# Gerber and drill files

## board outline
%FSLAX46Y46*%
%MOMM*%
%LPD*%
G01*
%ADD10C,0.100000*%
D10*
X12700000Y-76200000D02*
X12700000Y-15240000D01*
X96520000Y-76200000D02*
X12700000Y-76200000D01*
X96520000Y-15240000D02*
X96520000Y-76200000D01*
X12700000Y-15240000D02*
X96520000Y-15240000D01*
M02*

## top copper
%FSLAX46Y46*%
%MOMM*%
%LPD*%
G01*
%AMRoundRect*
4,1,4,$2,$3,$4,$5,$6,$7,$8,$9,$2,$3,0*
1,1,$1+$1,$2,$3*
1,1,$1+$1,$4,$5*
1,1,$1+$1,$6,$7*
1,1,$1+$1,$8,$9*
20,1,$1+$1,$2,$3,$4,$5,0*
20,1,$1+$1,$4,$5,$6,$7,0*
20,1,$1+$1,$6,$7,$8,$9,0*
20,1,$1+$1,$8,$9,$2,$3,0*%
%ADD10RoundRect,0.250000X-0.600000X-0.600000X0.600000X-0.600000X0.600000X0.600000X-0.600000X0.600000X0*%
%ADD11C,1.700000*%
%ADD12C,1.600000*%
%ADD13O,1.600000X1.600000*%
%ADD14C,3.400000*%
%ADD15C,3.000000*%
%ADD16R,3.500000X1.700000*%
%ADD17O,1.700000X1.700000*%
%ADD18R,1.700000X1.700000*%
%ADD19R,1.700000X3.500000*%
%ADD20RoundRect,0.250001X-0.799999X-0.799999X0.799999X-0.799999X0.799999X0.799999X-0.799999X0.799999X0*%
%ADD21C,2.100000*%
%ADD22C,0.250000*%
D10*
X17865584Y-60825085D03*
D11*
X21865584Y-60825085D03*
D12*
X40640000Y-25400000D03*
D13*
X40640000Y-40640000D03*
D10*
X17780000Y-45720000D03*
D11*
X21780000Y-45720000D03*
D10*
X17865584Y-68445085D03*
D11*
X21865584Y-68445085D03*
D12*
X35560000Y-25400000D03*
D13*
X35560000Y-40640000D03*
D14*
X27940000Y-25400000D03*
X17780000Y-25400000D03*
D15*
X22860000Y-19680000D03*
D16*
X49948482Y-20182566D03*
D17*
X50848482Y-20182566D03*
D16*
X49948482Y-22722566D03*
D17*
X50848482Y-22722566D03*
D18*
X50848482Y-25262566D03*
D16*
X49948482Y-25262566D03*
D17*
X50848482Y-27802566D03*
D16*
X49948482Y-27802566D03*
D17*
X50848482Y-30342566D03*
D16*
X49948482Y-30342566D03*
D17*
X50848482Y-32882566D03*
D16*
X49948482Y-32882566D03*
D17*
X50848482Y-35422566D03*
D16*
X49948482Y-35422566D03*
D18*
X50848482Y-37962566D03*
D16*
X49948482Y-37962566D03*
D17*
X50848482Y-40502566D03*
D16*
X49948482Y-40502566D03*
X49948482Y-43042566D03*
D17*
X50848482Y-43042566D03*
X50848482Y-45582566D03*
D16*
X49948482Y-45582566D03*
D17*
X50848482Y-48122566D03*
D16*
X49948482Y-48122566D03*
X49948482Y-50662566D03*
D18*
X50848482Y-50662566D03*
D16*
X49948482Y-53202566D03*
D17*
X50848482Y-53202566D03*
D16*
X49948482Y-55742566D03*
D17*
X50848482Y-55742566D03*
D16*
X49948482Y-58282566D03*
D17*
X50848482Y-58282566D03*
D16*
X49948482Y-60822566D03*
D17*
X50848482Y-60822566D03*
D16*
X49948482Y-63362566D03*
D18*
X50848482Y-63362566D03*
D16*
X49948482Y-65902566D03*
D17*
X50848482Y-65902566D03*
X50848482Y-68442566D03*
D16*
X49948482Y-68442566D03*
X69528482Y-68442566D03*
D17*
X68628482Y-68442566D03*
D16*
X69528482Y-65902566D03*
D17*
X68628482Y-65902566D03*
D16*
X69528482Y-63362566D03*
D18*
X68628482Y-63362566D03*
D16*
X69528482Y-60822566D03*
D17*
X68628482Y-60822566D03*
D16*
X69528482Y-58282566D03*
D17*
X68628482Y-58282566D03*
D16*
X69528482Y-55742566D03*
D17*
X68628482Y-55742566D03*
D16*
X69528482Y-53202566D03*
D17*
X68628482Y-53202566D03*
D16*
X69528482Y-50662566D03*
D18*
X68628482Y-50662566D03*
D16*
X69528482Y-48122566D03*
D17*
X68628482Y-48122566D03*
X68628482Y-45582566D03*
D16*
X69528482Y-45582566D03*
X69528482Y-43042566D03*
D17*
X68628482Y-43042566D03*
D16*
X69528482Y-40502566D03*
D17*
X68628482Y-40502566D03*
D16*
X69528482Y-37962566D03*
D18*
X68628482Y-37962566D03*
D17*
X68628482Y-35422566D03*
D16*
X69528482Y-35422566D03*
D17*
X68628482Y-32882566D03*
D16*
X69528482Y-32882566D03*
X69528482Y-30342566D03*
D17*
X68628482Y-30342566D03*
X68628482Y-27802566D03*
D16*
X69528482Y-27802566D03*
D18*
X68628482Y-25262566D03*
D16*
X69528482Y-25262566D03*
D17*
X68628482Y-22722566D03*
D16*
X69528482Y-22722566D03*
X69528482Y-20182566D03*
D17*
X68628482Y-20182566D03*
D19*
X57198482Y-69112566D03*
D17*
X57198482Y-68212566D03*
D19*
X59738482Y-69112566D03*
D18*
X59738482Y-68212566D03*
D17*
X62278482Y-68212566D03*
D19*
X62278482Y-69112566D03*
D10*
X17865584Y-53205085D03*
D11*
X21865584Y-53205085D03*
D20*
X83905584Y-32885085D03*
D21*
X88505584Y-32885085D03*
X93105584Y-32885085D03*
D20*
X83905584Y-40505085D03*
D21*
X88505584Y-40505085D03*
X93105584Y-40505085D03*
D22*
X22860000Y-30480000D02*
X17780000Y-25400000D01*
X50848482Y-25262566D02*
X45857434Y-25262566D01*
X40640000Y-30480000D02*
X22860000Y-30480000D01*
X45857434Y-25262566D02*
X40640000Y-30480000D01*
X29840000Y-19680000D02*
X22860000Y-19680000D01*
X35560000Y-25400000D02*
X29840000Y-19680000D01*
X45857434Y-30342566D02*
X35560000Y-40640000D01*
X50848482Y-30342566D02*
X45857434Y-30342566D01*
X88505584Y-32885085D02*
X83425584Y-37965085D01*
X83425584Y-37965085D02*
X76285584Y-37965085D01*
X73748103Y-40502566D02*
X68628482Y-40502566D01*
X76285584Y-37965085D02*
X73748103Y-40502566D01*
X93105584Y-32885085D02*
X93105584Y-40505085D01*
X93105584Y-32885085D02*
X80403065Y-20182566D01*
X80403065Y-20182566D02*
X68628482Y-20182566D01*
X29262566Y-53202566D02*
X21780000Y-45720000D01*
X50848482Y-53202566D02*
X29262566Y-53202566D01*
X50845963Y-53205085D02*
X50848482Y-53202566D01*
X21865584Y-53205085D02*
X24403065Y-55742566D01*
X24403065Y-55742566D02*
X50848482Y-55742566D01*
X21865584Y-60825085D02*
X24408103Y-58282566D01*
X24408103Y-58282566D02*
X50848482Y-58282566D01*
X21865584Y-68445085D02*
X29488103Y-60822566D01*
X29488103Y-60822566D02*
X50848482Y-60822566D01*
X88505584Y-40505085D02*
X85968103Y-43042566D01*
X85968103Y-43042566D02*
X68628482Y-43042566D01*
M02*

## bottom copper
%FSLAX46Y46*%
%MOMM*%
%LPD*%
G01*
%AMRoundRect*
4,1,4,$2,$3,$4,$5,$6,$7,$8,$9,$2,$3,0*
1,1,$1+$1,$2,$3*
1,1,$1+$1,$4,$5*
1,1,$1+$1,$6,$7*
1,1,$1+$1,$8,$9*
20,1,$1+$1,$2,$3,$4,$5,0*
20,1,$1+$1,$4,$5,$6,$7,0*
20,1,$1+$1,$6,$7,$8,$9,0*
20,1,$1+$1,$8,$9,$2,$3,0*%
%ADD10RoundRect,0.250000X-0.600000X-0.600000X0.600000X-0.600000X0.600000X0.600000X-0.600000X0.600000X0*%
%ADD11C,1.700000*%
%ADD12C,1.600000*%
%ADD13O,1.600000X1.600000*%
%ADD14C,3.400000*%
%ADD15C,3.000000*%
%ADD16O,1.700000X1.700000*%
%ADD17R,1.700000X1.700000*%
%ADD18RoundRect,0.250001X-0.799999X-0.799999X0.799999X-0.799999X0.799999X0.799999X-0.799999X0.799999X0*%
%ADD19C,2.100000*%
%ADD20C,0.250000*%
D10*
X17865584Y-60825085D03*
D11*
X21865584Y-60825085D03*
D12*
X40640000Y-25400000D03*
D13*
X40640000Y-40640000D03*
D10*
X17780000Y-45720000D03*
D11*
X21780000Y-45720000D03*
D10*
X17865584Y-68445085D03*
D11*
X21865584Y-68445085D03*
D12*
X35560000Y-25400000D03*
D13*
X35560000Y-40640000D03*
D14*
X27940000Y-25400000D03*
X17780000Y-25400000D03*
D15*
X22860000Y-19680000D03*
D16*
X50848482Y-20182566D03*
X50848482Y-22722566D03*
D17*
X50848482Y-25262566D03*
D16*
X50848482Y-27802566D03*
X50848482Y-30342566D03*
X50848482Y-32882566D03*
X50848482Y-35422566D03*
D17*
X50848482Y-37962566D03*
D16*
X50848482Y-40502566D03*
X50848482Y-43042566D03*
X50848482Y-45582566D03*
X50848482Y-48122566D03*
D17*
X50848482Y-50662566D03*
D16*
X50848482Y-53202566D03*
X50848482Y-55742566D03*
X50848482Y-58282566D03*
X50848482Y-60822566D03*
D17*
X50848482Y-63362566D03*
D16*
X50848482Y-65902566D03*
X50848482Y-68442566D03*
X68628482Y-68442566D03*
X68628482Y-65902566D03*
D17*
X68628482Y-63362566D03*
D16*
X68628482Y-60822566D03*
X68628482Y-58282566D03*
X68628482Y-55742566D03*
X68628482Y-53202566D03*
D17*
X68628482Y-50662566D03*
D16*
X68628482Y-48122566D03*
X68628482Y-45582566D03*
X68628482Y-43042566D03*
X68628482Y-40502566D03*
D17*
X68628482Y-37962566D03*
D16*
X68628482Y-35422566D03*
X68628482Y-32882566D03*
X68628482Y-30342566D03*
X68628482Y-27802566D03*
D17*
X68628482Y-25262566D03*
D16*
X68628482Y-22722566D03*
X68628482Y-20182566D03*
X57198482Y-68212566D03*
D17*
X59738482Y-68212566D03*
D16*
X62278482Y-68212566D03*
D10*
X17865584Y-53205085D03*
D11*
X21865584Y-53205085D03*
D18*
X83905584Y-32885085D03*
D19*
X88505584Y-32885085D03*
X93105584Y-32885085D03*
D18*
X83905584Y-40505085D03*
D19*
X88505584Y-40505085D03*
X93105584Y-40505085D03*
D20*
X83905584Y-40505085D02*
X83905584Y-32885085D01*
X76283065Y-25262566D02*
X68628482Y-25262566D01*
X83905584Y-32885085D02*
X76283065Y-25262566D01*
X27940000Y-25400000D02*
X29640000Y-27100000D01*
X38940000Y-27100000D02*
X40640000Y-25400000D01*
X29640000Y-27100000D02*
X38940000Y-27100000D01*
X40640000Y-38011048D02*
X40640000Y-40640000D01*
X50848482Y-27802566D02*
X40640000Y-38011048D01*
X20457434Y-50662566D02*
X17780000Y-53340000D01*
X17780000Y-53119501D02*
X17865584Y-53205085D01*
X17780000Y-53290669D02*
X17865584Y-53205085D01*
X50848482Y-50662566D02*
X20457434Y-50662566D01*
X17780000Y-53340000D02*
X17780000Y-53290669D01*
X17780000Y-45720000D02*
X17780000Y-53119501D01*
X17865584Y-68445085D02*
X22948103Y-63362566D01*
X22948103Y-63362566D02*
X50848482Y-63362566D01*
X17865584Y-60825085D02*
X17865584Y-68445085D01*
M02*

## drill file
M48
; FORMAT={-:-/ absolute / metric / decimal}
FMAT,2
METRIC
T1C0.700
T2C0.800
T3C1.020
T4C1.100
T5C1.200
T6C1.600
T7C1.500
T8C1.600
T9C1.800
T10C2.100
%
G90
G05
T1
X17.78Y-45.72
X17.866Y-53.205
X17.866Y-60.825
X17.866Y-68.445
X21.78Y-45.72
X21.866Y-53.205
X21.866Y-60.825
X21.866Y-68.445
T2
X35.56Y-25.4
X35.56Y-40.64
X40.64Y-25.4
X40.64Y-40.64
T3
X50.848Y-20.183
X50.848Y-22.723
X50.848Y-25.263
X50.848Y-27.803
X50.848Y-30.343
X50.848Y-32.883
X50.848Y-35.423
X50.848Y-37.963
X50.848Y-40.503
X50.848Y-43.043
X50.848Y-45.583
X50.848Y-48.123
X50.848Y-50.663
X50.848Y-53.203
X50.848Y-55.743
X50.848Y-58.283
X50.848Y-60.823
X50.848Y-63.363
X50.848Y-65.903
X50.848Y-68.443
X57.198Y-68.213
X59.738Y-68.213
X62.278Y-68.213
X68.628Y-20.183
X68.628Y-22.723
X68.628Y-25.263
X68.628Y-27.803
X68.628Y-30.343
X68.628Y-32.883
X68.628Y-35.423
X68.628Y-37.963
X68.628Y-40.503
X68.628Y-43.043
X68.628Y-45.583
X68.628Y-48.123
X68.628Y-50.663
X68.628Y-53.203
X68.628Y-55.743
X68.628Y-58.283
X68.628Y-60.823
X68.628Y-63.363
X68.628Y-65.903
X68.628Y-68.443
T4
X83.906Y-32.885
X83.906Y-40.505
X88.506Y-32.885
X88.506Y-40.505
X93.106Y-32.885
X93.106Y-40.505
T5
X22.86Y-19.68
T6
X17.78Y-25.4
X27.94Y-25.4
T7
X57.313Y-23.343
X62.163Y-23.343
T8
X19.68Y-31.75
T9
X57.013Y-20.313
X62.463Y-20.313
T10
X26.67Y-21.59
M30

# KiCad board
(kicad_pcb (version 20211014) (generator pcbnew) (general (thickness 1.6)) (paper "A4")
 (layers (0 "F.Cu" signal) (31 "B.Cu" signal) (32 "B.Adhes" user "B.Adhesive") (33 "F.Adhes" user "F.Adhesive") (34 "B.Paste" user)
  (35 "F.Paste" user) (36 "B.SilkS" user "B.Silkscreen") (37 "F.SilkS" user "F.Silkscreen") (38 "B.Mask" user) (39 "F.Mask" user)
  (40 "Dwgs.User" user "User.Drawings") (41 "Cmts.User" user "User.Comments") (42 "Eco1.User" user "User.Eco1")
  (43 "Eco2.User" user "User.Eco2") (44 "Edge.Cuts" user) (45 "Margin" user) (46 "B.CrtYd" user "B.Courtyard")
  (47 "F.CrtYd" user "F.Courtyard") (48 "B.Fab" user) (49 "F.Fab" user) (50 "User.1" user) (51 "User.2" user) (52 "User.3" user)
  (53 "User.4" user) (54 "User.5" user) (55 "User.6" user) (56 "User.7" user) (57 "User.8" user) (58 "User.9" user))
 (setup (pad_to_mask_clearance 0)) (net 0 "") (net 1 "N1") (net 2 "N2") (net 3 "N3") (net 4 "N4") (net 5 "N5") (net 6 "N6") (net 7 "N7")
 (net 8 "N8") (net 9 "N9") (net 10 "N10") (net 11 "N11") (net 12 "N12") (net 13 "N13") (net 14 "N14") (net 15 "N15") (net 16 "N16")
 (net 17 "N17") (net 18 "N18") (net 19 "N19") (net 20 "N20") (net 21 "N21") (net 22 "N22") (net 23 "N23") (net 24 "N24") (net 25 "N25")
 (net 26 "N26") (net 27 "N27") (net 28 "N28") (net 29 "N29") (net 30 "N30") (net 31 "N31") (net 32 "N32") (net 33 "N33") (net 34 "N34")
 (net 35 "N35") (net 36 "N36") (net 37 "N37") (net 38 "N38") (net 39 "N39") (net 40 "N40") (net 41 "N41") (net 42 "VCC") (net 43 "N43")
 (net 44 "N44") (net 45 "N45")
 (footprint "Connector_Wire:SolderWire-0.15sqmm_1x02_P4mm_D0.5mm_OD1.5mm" (layer "F.Cu") (at 17.865584 60.825085)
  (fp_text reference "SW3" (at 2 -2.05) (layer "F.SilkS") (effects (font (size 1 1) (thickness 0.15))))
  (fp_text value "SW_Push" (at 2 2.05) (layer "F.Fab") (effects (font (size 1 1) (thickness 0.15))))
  (pad "1" thru_hole roundrect (at 0 0) (size 1.7 1.7) (drill 0.7) (layers *.Cu *.Mask) (roundrect_rratio 0.147059) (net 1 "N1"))
  (pad "2" thru_hole circle (at 4 0) (size 1.7 1.7) (drill 0.7) (layers *.Cu *.Mask) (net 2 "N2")))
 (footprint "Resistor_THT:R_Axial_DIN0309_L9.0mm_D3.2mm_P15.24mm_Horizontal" (layer "F.Cu") (at 40.64 25.4 -90)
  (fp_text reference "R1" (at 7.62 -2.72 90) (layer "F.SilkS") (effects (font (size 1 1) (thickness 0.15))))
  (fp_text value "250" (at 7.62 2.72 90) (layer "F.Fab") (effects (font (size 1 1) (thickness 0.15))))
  (pad "1" thru_hole circle (at 0 0 270) (size 1.6 1.6) (drill 0.8) (layers *.Cu *.Mask) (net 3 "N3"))
  (pad "2" thru_hole oval (at 15.24 0 270) (size 1.6 1.6) (drill 0.8) (layers *.Cu *.Mask) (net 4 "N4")))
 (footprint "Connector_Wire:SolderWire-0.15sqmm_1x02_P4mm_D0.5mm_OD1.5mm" (layer "F.Cu") (at 17.78 45.72)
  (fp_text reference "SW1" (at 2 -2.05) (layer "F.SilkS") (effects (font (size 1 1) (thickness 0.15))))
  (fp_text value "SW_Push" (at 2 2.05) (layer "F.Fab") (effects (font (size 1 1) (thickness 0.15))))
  (pad "1" thru_hole roundrect (at 0 0) (size 1.7 1.7) (drill 0.7) (layers *.Cu *.Mask) (roundrect_rratio 0.147059) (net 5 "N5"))
  (pad "2" thru_hole circle (at 4 0) (size 1.7 1.7) (drill 0.7) (layers *.Cu *.Mask) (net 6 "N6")))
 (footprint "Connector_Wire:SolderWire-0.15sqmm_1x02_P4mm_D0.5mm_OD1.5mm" (layer "F.Cu") (at 17.865584 68.445085)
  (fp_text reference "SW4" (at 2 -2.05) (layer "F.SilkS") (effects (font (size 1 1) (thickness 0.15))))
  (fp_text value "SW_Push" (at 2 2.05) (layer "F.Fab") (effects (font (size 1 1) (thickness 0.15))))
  (pad "1" thru_hole roundrect (at 0 0) (size 1.7 1.7) (drill 0.7) (layers *.Cu *.Mask) (roundrect_rratio 0.147059) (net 1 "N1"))
  (pad "2" thru_hole circle (at 4 0) (size 1.7 1.7) (drill 0.7) (layers *.Cu *.Mask) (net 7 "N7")))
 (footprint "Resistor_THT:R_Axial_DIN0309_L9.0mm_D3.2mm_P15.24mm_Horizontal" (layer "F.Cu") (at 35.56 25.4 -90)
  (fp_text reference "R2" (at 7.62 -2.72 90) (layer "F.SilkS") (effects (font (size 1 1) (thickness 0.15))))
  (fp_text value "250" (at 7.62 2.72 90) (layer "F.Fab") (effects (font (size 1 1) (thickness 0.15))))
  (pad "1" thru_hole circle (at 0 0 270) (size 1.6 1.6) (drill 0.8) (layers *.Cu *.Mask) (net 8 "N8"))
  (pad "2" thru_hole oval (at 15.24 0 270) (size 1.6 1.6) (drill 0.8) (layers *.Cu *.Mask) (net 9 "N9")))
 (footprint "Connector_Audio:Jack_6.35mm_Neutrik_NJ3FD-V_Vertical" (layer "F.Cu") (at 22.86 19.68)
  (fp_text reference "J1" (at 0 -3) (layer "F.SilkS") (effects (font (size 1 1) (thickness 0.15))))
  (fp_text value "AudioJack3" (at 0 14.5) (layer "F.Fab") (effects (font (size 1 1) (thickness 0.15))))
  (pad "" np_thru_hole circle (at 3.81 1.91 180) (size 2.1 2.1) (drill 2.1) (layers *.Cu *.Mask))
  (pad "" np_thru_hole circle (at -3.18 12.07 180) (size 1.6 1.6) (drill 1.6) (layers *.Cu *.Mask))
  (pad "R" thru_hole circle (at 5.08 5.72 180) (size 3.4 3.4) (drill 1.6) (layers *.Cu *.Mask) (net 3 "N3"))
  (pad "S" thru_hole circle (at -5.08 5.72 180) (size 3.4 3.4) (drill 1.6) (layers *.Cu *.Mask) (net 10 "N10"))
  (pad "T" thru_hole circle (at 0 0 180) (size 3 3) (drill 1.2) (layers *.Cu *.Mask) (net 8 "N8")))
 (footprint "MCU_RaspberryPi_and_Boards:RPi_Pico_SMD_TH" (layer "F.Cu") (at 59.738482 44.312566)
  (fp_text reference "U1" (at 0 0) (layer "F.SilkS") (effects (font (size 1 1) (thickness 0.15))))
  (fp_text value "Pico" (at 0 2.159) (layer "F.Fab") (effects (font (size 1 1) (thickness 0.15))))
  (pad "" np_thru_hole oval (at -2.725 -24) (size 1.8 1.8) (drill 1.8) (layers *.Cu *.Mask))
  (pad "" np_thru_hole oval (at -2.425 -20.97) (size 1.5 1.5) (drill 1.5) (layers *.Cu *.Mask))
  (pad "" np_thru_hole oval (at 2.425 -20.97) (size 1.5 1.5) (drill 1.5) (layers *.Cu *.Mask))
  (pad "" np_thru_hole oval (at 2.725 -24) (size 1.8 1.8) (drill 1.8) (layers *.Cu *.Mask))
  (pad "1" smd rect (at -8.89 -24.13) (size 3.5 1.7) (drill (offset -0.9 0)) (layers "F.Cu" "F.Mask") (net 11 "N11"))
  (pad "1" thru_hole oval (at -8.89 -24.13) (size 1.7 1.7) (drill 1.02) (layers *.Cu *.Mask) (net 11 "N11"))
  (pad "2" smd rect (at -8.89 -21.59) (size 3.5 1.7) (drill (offset -0.9 0)) (layers "F.Cu" "F.Mask") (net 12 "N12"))
  (pad "2" thru_hole oval (at -8.89 -21.59) (size 1.7 1.7) (drill 1.02) (layers *.Cu *.Mask) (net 12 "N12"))
  (pad "3" thru_hole rect (at -8.89 -19.05) (size 1.7 1.7) (drill 1.02) (layers *.Cu *.Mask) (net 10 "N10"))
  (pad "3" smd rect (at -8.89 -19.05) (size 3.5 1.7) (drill (offset -0.9 0)) (layers "F.Cu" "F.Mask") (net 10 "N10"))
  (pad "4" thru_hole oval (at -8.89 -16.51) (size 1.7 1.7) (drill 1.02) (layers *.Cu *.Mask) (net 4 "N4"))
  (pad "4" smd rect (at -8.89 -16.51) (size 3.5 1.7) (drill (offset -0.9 0)) (layers "F.Cu" "F.Mask") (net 4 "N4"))
  (pad "5" thru_hole oval (at -8.89 -13.97) (size 1.7 1.7) (drill 1.02) (layers *.Cu *.Mask) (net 9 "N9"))
  (pad "5" smd rect (at -8.89 -13.97) (size 3.5 1.7) (drill (offset -0.9 0)) (layers "F.Cu" "F.Mask") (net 9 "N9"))
  (pad "6" thru_hole oval (at -8.89 -11.43) (size 1.7 1.7) (drill 1.02) (layers *.Cu *.Mask) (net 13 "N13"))
  (pad "6" smd rect (at -8.89 -11.43) (size 3.5 1.7) (drill (offset -0.9 0)) (layers "F.Cu" "F.Mask") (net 13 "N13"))
  (pad "7" thru_hole oval (at -8.89 -8.89) (size 1.7 1.7) (drill 1.02) (layers *.Cu *.Mask) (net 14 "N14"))
  (pad "7" smd rect (at -8.89 -8.89) (size 3.5 1.7) (drill (offset -0.9 0)) (layers "F.Cu" "F.Mask") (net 14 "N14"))
  (pad "8" thru_hole rect (at -8.89 -6.35) (size 1.7 1.7) (drill 1.02) (layers *.Cu *.Mask) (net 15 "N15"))
  (pad "8" smd rect (at -8.89 -6.35) (size 3.5 1.7) (drill (offset -0.9 0)) (layers "F.Cu" "F.Mask") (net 15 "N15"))
  (pad "9" thru_hole oval (at -8.89 -3.81) (size 1.7 1.7) (drill 1.02) (layers *.Cu *.Mask) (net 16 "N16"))
  (pad "9" smd rect (at -8.89 -3.81) (size 3.5 1.7) (drill (offset -0.9 0)) (layers "F.Cu" "F.Mask") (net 16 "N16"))
  (pad "10" smd rect (at -8.89 -1.27) (size 3.5 1.7) (drill (offset -0.9 0)) (layers "F.Cu" "F.Mask") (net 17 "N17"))
  (pad "10" thru_hole oval (at -8.89 -1.27) (size 1.7 1.7) (drill 1.02) (layers *.Cu *.Mask) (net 17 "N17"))
  (pad "11" thru_hole oval (at -8.89 1.27) (size 1.7 1.7) (drill 1.02) (layers *.Cu *.Mask) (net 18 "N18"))
  (pad "11" smd rect (at -8.89 1.27) (size 3.5 1.7) (drill (offset -0.9 0)) (layers "F.Cu" "F.Mask") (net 18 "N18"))
  (pad "12" thru_hole oval (at -8.89 3.81) (size 1.7 1.7) (drill 1.02) (layers *.Cu *.Mask) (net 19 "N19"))
  (pad "12" smd rect (at -8.89 3.81) (size 3.5 1.7) (drill (offset -0.9 0)) (layers "F.Cu" "F.Mask") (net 19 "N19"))
  (pad "13" smd rect (at -8.89 6.35) (size 3.5 1.7) (drill (offset -0.9 0)) (layers "F.Cu" "F.Mask") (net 5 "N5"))
  (pad "13" thru_hole rect (at -8.89 6.35) (size 1.7 1.7) (drill 1.02) (layers *.Cu *.Mask) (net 5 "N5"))
  (pad "14" smd rect (at -8.89 8.89) (size 3.5 1.7) (drill (offset -0.9 0)) (layers "F.Cu" "F.Mask") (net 6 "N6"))
  (pad "14" thru_hole oval (at -8.89 8.89) (size 1.7 1.7) (drill 1.02) (layers *.Cu *.Mask) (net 6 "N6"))
  (pad "15" smd rect (at -8.89 11.43) (size 3.5 1.7) (drill (offset -0.9 0)) (layers "F.Cu" "F.Mask") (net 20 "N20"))
  (pad "15" thru_hole oval (at -8.89 11.43) (size 1.7 1.7) (drill 1.02) (layers *.Cu *.Mask) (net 20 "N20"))
  (pad "16" smd rect (at -8.89 13.97) (size 3.5 1.7) (drill (offset -0.9 0)) (layers "F.Cu" "F.Mask") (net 2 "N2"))
  (pad "16" thru_hole oval (at -8.89 13.97) (size 1.7 1.7) (drill 1.02) (layers *.Cu *.Mask) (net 2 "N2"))
  (pad "17" smd rect (at -8.89 16.51) (size 3.5 1.7) (drill (offset -0.9 0)) (layers "F.Cu" "F.Mask") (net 7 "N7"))
  (pad "17" thru_hole oval (at -8.89 16.51) (size 1.7 1.7) (drill 1.02) (layers *.Cu *.Mask) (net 7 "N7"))
  (pad "18" smd rect (at -8.89 19.05) (size 3.5 1.7) (drill (offset -0.9 0)) (layers "F.Cu" "F.Mask") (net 1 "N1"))
  (pad "18" thru_hole rect (at -8.89 19.05) (size 1.7 1.7) (drill 1.02) (layers *.Cu *.Mask) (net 1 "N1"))
  (pad "19" smd rect (at -8.89 21.59) (size 3.5 1.7) (drill (offset -0.9 0)) (layers "F.Cu" "F.Mask") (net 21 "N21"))
  (pad "19" thru_hole oval (at -8.89 21.59) (size 1.7 1.7) (drill 1.02) (layers *.Cu *.Mask) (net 21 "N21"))
  (pad "20" thru_hole oval (at -8.89 24.13) (size 1.7 1.7) (drill 1.02) (layers *.Cu *.Mask) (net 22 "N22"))
  (pad "20" smd rect (at -8.89 24.13) (size 3.5 1.7) (drill (offset -0.9 0)) (layers "F.Cu" "F.Mask") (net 22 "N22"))
  (pad "21" smd rect (at 8.89 24.13) (size 3.5 1.7) (drill (offset 0.9 0)) (layers "F.Cu" "F.Mask") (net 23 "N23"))
  (pad "21" thru_hole oval (at 8.89 24.13) (size 1.7 1.7) (drill 1.02) (layers *.Cu *.Mask) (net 23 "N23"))
  (pad "22" smd rect (at 8.89 21.59) (size 3.5 1.7) (drill (offset 0.9 0)) (layers "F.Cu" "F.Mask") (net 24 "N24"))
  (pad "22" thru_hole oval (at 8.89 21.59) (size 1.7 1.7) (drill 1.02) (layers *.Cu *.Mask) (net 24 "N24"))
  (pad "23" smd rect (at 8.89 19.05) (size 3.5 1.7) (drill (offset 0.9 0)) (layers "F.Cu" "F.Mask") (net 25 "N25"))
  (pad "23" thru_hole rect (at 8.89 19.05) (size 1.7 1.7) (drill 1.02) (layers *.Cu *.Mask) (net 25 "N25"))
  (pad "24" smd rect (at 8.89 16.51) (size 3.5 1.7) (drill (offset 0.9 0)) (layers "F.Cu" "F.Mask") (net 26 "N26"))
  (pad "24" thru_hole oval (at 8.89 16.51) (size 1.7 1.7) (drill 1.02) (layers *.Cu *.Mask) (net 26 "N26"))
  (pad "25" smd rect (at 8.89 13.97) (size 3.5 1.7) (drill (offset 0.9 0)) (layers "F.Cu" "F.Mask") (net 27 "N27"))
  (pad "25" thru_hole oval (at 8.89 13.97) (size 1.7 1.7) (drill 1.02) (layers *.Cu *.Mask) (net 27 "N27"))
  (pad "26" smd rect (at 8.89 11.43) (size 3.5 1.7) (drill (offset 0.9 0)) (layers "F.Cu" "F.Mask") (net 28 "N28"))
  (pad "26" thru_hole oval (at 8.89 11.43) (size 1.7 1.7) (drill 1.02) (layers *.Cu *.Mask) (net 28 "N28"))
  (pad "27" smd rect (at 8.89 8.89) (size 3.5 1.7) (drill (offset 0.9 0)) (layers "F.Cu" "F.Mask") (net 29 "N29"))
  (pad "27" thru_hole oval (at 8.89 8.89) (size 1.7 1.7) (drill 1.02) (layers *.Cu *.Mask) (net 29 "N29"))
  (pad "28" smd rect (at 8.89 6.35) (size 3.5 1.7) (drill (offset 0.9 0)) (layers "F.Cu" "F.Mask") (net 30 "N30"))
  (pad "28" thru_hole rect (at 8.89 6.35) (size 1.7 1.7) (drill 1.02) (layers *.Cu *.Mask) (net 30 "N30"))
  (pad "29" smd rect (at 8.89 3.81) (size 3.5 1.7) (drill (offset 0.9 0)) (layers "F.Cu" "F.Mask") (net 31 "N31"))
  (pad "29" thru_hole oval (at 8.89 3.81) (size 1.7 1.7) (drill 1.02) (layers *.Cu *.Mask) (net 31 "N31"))
  (pad "30" thru_hole oval (at 8.89 1.27) (size 1.7 1.7) (drill 1.02) (layers *.Cu *.Mask) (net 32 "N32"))
  (pad "30" smd rect (at 8.89 1.27) (size 3.5 1.7) (drill (offset 0.9 0)) (layers "F.Cu" "F.Mask") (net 32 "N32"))
  (pad "31" smd rect (at 8.89 -1.27) (size 3.5 1.7) (drill (offset 0.9 0)) (layers "F.Cu" "F.Mask") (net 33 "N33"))
  (pad "31" thru_hole oval (at 8.89 -1.27) (size 1.7 1.7) (drill 1.02) (layers *.Cu *.Mask) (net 33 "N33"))
  (pad "32" smd rect (at 8.89 -3.81) (size 3.5 1.7) (drill (offset 0.9 0)) (layers "F.Cu" "F.Mask") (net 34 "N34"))
  (pad "32" thru_hole oval (at 8.89 -3.81) (size 1.7 1.7) (drill 1.02) (layers *.Cu *.Mask) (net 34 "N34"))
  (pad "33" smd rect (at 8.89 -6.35) (size 3.5 1.7) (drill (offset 0.9 0)) (layers "F.Cu" "F.Mask") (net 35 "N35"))
  (pad "33" thru_hole rect (at 8.89 -6.35) (size 1.7 1.7) (drill 1.02) (layers *.Cu *.Mask) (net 35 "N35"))
  (pad "34" thru_hole oval (at 8.89 -8.89) (size 1.7 1.7) (drill 1.02) (layers *.Cu *.Mask) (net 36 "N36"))
  (pad "34" smd rect (at 8.89 -8.89) (size 3.5 1.7) (drill (offset 0.9 0)) (layers "F.Cu" "F.Mask") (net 36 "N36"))
  (pad "35" thru_hole oval (at 8.89 -11.43) (size 1.7 1.7) (drill 1.02) (layers *.Cu *.Mask) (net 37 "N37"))
  (pad "35" smd rect (at 8.89 -11.43) (size 3.5 1.7) (drill (offset 0.9 0)) (layers "F.Cu" "F.Mask") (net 37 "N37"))
  (pad "36" smd rect (at 8.89 -13.97) (size 3.5 1.7) (drill (offset 0.9 0)) (layers "F.Cu" "F.Mask") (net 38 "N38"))
  (pad "36" thru_hole oval (at 8.89 -13.97) (size 1.7 1.7) (drill 1.02) (layers *.Cu *.Mask) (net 38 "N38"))
  (pad "37" thru_hole oval (at 8.89 -16.51) (size 1.7 1.7) (drill 1.02) (layers *.Cu *.Mask) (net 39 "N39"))
  (pad "37" smd rect (at 8.89 -16.51) (size 3.5 1.7) (drill (offset 0.9 0)) (layers "F.Cu" "F.Mask") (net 39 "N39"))
  (pad "38" thru_hole rect (at 8.89 -19.05) (size 1.7 1.7) (drill 1.02) (layers *.Cu *.Mask) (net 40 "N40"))
  (pad "38" smd rect (at 8.89 -19.05) (size 3.5 1.7) (drill (offset 0.9 0)) (layers "F.Cu" "F.Mask") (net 40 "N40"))
  (pad "39" thru_hole oval (at 8.89 -21.59) (size 1.7 1.7) (drill 1.02) (layers *.Cu *.Mask) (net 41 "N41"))
  (pad "39" smd rect (at 8.89 -21.59) (size 3.5 1.7) (drill (offset 0.9 0)) (layers "F.Cu" "F.Mask") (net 41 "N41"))
  (pad "40" smd rect (at 8.89 -24.13) (size 3.5 1.7) (drill (offset 0.9 0)) (layers "F.Cu" "F.Mask") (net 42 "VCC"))
  (pad "40" thru_hole oval (at 8.89 -24.13) (size 1.7 1.7) (drill 1.02) (layers *.Cu *.Mask) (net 42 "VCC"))
  (pad "41" smd rect (at -2.54 23.9 90) (size 3.5 1.7) (drill (offset -0.9 0)) (layers "F.Cu" "F.Mask") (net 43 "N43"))
  (pad "41" thru_hole oval (at -2.54 23.9) (size 1.7 1.7) (drill 1.02) (layers *.Cu *.Mask) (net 43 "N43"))
  (pad "42" smd rect (at 0 23.9 90) (size 3.5 1.7) (drill (offset -0.9 0)) (layers "F.Cu" "F.Mask") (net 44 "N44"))
  (pad "42" thru_hole rect (at 0 23.9) (size 1.7 1.7) (drill 1.02) (layers *.Cu *.Mask) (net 44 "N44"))
  (pad "43" thru_hole oval (at 2.54 23.9) (size 1.7 1.7) (drill 1.02) (layers *.Cu *.Mask) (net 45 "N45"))
  (pad "43" smd rect (at 2.54 23.9 90) (size 3.5 1.7) (drill (offset -0.9 0)) (layers "F.Cu" "F.Mask") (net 45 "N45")))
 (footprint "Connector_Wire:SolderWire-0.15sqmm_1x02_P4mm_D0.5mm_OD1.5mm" (layer "F.Cu") (at 17.865584 53.205085)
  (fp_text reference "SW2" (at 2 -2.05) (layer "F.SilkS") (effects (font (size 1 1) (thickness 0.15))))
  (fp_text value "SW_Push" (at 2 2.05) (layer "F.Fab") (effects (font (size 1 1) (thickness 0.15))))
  (pad "1" thru_hole roundrect (at 0 0) (size 1.7 1.7) (drill 0.7) (layers *.Cu *.Mask) (roundrect_rratio 0.147059) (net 5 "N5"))
  (pad "2" thru_hole circle (at 4 0) (size 1.7 1.7) (drill 0.7) (layers *.Cu *.Mask) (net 20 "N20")))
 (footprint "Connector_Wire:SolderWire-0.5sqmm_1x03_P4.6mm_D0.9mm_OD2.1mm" (layer "F.Cu") (at 83.905584 32.885085)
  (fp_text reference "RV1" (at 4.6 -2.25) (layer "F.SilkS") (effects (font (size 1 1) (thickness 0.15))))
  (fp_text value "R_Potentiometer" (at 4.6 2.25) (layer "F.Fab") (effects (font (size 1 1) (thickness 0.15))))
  (pad "1" thru_hole roundrect (at 0 0) (size 2.1 2.1) (drill 1.1) (layers *.Cu *.Mask) (roundrect_rratio 0.119048) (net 40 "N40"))
  (pad "2" thru_hole circle (at 4.6 0) (size 2.1 2.1) (drill 1.1) (layers *.Cu *.Mask) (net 34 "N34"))
  (pad "3" thru_hole circle (at 9.2 0) (size 2.1 2.1) (drill 1.1) (layers *.Cu *.Mask) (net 42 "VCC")))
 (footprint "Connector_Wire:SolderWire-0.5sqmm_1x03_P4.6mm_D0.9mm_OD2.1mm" (layer "F.Cu") (at 83.905584 40.505085)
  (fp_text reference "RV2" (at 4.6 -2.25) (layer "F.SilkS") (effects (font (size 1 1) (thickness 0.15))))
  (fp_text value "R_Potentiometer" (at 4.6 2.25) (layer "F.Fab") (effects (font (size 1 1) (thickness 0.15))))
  (pad "1" thru_hole roundrect (at 0 0) (size 2.1 2.1) (drill 1.1) (layers *.Cu *.Mask) (roundrect_rratio 0.119048) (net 40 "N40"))
  (pad "2" thru_hole circle (at 4.6 0) (size 2.1 2.1) (drill 1.1) (layers *.Cu *.Mask) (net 33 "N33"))
  (pad "3" thru_hole circle (at 9.2 0) (size 2.1 2.1) (drill 1.1) (layers *.Cu *.Mask) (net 42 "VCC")))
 (gr_line (start 12.7 76.2) (end 12.7 15.24) (layer "Edge.Cuts") (width 0.1))
 (gr_line (start 96.52 76.2) (end 12.7 76.2) (layer "Edge.Cuts") (width 0.1))
 (gr_line (start 96.52 15.24) (end 96.52 76.2) (layer "Edge.Cuts") (width 0.1))
 (gr_line (start 12.7 15.24) (end 96.52 15.24) (layer "Edge.Cuts") (width 0.1))
 (segment (start 22.86 30.48) (end 17.78 25.4) (width 0.25) (layer "F.Cu") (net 10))
 (segment (start 50.848482 25.262566) (end 45.857434 25.262566) (width 0.25) (layer "F.Cu") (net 10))
 (segment (start 40.64 30.48) (end 22.86 30.48) (width 0.25) (layer "F.Cu") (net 10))
 (segment (start 45.857434 25.262566) (end 40.64 30.48) (width 0.25) (layer "F.Cu") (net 10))
 (segment (start 83.905584 40.505085) (end 83.905584 32.885085) (width 0.25) (layer "B.Cu") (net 40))
 (segment (start 76.283065 25.262566) (end 68.628482 25.262566) (width 0.25) (layer "B.Cu") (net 40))
 (segment (start 83.905584 32.885085) (end 76.283065 25.262566) (width 0.25) (layer "B.Cu") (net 40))
 (segment (start 27.94 25.4) (end 29.64 27.1) (width 0.25) (layer "B.Cu") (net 3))
 (segment (start 38.94 27.1) (end 40.64 25.4) (width 0.25) (layer "B.Cu") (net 3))
 (segment (start 29.64 27.1) (end 38.94 27.1) (width 0.25) (layer "B.Cu") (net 3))
 (segment (start 29.84 19.68) (end 22.86 19.68) (width 0.25) (layer "F.Cu") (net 8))
 (segment (start 35.56 25.4) (end 29.84 19.68) (width 0.25) (layer "F.Cu") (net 8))
 (segment (start 40.64 38.011048) (end 40.64 40.64) (width 0.25) (layer "B.Cu") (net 4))
 (segment (start 50.848482 27.802566) (end 40.64 38.011048) (width 0.25) (layer "B.Cu") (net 4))
 (segment (start 45.857434 30.342566) (end 35.56 40.64) (width 0.25) (layer "F.Cu") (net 9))
 (segment (start 50.848482 30.342566) (end 45.857434 30.342566) (width 0.25) (layer "F.Cu") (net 9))
 (segment (start 88.505584 32.885085) (end 83.425584 37.965085) (width 0.25) (layer "F.Cu") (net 34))
 (segment (start 83.425584 37.965085) (end 76.285584 37.965085) (width 0.25) (layer "F.Cu") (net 34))
 (segment (start 73.748103 40.502566) (end 68.628482 40.502566) (width 0.25) (layer "F.Cu") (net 34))
 (segment (start 76.285584 37.965085) (end 73.748103 40.502566) (width 0.25) (layer "F.Cu") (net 34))
 (segment (start 93.105584 32.885085) (end 93.105584 40.505085) (width 0.25) (layer "F.Cu") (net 42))
 (segment (start 93.105584 32.885085) (end 80.403065 20.182566) (width 0.25) (layer "F.Cu") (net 42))
 (segment (start 80.403065 20.182566) (end 68.628482 20.182566) (width 0.25) (layer "F.Cu") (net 42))
 (segment (start 20.457434 50.662566) (end 17.78 53.34) (width 0.25) (layer "B.Cu") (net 5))
 (segment (start 17.78 53.119501) (end 17.865584 53.205085) (width 0.25) (layer "B.Cu") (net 5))
 (segment (start 17.78 53.290669) (end 17.865584 53.205085) (width 0.25) (layer "B.Cu") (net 5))
 (segment (start 50.848482 50.662566) (end 20.457434 50.662566) (width 0.25) (layer "B.Cu") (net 5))
 (segment (start 17.78 53.34) (end 17.78 53.290669) (width 0.25) (layer "B.Cu") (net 5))
 (segment (start 17.78 45.72) (end 17.78 53.119501) (width 0.25) (layer "B.Cu") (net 5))
 (segment (start 29.262566 53.202566) (end 21.78 45.72) (width 0.25) (layer "F.Cu") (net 6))
 (segment (start 50.848482 53.202566) (end 29.262566 53.202566) (width 0.25) (layer "F.Cu") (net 6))
 (segment (start 50.845963 53.205085) (end 50.848482 53.202566) (width 0.25) (layer "F.Cu") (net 6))
 (segment (start 21.865584 53.205085) (end 24.403065 55.742566) (width 0.25) (layer "F.Cu") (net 20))
 (segment (start 24.403065 55.742566) (end 50.848482 55.742566) (width 0.25) (layer "F.Cu") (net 20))
 (segment (start 21.865584 60.825085) (end 24.408103 58.282566) (width 0.25) (layer "F.Cu") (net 2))
 (segment (start 24.408103 58.282566) (end 50.848482 58.282566) (width 0.25) (layer "F.Cu") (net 2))
 (segment (start 21.865584 68.445085) (end 29.488103 60.822566) (width 0.25) (layer "F.Cu") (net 7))
 (segment (start 29.488103 60.822566) (end 50.848482 60.822566) (width 0.25) (layer "F.Cu") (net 7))
 (segment (start 88.505584 40.505085) (end 85.968103 43.042566) (width 0.25) (layer "F.Cu") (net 33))
 (segment (start 85.968103 43.042566) (end 68.628482 43.042566) (width 0.25) (layer "F.Cu") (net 33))
 (segment (start 17.865584 68.445085) (end 22.948103 63.362566) (width 0.25) (layer "B.Cu") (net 1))
 (segment (start 22.948103 63.362566) (end 50.848482 63.362566) (width 0.25) (layer "B.Cu") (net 1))
 (segment (start 17.865584 60.825085) (end 17.865584 68.445085) (width 0.25) (layer "B.Cu") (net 1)))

